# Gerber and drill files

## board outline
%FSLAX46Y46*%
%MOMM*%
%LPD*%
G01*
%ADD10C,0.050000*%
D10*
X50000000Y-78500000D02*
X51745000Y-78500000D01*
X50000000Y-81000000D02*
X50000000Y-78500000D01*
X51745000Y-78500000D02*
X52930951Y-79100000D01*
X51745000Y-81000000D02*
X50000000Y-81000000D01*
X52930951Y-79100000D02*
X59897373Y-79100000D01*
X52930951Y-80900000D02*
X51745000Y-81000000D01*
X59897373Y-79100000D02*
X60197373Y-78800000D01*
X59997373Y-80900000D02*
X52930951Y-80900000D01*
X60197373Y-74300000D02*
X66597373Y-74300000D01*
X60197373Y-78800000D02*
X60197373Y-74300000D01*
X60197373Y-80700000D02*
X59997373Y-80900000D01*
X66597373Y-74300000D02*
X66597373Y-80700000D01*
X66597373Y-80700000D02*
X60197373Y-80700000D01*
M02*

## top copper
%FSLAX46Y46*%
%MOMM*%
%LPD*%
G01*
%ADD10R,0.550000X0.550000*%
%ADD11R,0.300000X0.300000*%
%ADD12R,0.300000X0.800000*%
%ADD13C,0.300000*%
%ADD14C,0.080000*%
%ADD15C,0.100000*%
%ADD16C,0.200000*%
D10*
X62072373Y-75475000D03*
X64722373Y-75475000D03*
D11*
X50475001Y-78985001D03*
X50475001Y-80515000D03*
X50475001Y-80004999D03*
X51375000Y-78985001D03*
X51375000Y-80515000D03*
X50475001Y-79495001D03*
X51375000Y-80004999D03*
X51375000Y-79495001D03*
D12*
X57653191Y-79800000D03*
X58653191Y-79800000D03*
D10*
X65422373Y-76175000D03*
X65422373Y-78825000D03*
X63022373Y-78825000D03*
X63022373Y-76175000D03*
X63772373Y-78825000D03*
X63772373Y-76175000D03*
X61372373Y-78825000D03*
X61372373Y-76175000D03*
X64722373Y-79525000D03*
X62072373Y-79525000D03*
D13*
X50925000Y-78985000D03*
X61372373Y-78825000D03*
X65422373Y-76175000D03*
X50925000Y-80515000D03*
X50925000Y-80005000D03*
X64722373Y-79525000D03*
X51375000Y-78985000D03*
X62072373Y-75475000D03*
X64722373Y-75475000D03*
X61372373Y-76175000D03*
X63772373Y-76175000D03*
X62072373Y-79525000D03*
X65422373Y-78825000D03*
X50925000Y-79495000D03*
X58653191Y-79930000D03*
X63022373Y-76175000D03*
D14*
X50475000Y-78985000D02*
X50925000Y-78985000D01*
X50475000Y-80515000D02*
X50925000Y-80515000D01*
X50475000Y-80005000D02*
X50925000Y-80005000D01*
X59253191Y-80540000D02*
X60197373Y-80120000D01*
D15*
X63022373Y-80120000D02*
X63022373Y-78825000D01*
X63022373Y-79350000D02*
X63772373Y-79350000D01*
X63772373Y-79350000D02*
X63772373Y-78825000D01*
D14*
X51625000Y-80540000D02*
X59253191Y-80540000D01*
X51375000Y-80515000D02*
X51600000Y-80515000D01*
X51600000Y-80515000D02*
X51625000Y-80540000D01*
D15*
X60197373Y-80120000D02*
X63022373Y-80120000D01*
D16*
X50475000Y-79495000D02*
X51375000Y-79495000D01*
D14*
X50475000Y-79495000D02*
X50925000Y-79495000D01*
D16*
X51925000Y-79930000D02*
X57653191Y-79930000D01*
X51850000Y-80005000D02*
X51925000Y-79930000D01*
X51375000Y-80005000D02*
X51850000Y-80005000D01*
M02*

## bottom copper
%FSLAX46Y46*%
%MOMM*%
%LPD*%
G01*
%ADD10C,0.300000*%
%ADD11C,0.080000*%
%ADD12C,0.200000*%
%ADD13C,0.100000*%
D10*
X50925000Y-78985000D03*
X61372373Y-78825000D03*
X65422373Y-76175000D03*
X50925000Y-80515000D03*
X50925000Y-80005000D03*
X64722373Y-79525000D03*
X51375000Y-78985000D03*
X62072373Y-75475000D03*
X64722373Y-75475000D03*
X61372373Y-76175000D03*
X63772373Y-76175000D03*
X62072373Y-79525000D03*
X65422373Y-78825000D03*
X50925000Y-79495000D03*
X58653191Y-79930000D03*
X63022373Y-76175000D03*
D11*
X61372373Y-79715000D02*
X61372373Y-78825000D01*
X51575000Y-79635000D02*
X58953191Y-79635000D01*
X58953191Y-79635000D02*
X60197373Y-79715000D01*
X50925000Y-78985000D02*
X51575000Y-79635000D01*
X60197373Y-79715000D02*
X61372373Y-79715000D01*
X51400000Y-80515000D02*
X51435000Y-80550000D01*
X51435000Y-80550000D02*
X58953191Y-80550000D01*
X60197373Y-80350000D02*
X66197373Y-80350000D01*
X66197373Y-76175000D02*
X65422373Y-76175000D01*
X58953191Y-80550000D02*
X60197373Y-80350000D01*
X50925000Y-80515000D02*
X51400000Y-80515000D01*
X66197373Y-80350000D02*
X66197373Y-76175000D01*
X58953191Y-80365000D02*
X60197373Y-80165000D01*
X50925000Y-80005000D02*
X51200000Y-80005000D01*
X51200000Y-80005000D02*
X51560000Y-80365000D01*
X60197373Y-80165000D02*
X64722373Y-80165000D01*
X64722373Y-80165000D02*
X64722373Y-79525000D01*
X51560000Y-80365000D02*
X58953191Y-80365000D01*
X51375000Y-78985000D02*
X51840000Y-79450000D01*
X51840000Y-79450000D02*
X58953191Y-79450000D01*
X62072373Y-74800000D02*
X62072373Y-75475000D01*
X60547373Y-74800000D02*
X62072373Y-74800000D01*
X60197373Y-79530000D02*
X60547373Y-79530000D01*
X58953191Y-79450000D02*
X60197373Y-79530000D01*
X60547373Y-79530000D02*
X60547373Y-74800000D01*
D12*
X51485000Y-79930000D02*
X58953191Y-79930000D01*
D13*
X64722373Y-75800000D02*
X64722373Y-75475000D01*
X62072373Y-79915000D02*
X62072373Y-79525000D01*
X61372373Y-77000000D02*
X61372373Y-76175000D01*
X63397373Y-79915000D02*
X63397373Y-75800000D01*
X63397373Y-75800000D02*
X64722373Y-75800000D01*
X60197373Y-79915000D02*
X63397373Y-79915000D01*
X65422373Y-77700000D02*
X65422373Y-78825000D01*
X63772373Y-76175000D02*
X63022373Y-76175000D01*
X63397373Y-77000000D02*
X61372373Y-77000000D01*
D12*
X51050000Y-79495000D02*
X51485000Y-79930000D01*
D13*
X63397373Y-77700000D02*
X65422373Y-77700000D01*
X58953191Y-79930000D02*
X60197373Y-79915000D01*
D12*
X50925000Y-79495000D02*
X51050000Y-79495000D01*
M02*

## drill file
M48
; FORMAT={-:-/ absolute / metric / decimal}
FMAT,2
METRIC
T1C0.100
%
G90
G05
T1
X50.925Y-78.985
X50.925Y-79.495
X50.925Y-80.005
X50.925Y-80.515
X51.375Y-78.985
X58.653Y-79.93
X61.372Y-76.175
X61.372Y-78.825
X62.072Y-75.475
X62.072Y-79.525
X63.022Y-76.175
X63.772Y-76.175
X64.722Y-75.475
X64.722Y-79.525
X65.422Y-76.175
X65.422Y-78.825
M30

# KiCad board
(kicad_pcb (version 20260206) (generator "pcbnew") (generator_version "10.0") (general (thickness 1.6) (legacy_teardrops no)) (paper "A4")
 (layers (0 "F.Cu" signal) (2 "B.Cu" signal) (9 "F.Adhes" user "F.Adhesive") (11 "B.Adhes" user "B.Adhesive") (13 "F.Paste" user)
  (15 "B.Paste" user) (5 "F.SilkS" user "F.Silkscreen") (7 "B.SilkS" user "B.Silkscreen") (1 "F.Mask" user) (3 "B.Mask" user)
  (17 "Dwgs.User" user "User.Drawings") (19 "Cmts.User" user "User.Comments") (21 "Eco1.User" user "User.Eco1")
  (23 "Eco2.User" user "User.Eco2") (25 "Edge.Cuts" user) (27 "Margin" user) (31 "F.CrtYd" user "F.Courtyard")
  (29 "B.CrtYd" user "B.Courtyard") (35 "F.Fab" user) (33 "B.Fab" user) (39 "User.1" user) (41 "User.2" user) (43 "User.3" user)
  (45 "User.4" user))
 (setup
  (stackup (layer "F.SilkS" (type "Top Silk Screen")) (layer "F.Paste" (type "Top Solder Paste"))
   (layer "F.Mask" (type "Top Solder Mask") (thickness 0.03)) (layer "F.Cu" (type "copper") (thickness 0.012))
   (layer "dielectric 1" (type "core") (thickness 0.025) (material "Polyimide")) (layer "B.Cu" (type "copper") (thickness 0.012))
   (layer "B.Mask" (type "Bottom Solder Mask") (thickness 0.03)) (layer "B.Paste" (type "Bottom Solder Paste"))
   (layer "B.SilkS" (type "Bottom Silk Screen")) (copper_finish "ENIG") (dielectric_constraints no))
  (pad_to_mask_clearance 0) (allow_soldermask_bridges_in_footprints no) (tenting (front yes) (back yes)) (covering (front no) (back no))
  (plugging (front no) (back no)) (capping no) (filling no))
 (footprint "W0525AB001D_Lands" (layer "F.Cu") (at 58.153191 79.93)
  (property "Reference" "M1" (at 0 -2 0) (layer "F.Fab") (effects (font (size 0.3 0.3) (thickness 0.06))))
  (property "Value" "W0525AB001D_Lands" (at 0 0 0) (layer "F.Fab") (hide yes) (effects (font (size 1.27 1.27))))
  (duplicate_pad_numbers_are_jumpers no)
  (pad "1" smd rect (at -0.5 -0.13) (size 0.3 0.8) (layers "F.Cu" "F.Mask") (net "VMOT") (solder_mask_margin 0.05) (thermal_bridge_angle 45))
  (pad "2" smd rect (at 0.5 -0.13) (size 0.3 0.8) (layers "F.Cu" "F.Mask") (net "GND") (solder_mask_margin 0.05) (thermal_bridge_angle 45)))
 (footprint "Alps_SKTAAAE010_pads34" (layer "F.Cu") (at 63.397373 79.9 180)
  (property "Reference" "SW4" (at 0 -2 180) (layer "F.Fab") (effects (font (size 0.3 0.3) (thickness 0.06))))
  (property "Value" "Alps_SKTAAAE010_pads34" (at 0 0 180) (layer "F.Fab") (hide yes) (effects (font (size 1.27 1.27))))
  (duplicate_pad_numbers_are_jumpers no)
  (pad "3" smd rect (at -1.325 0.375 180) (size 0.55 0.55) (layers "F.Cu" "F.Mask" "F.Paste") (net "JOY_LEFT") (solder_mask_margin 0.05)
   (thermal_bridge_angle 45))
  (pad "4" smd rect (at 1.325 0.375 180) (size 0.55 0.55) (layers "F.Cu" "F.Mask" "F.Paste") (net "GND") (solder_mask_margin 0.05)
   (thermal_bridge_angle 45)))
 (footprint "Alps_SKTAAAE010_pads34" (layer "F.Cu") (at 60.997373 77.5 90)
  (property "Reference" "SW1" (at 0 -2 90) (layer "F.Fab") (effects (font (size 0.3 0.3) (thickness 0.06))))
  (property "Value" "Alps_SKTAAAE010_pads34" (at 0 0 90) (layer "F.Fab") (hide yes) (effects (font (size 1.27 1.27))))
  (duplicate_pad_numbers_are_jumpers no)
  (pad "3" smd rect (at -1.325 0.375 90) (size 0.55 0.55) (layers "F.Cu" "F.Mask" "F.Paste") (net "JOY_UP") (solder_mask_margin 0.05)
   (thermal_bridge_angle 45))
  (pad "4" smd rect (at 1.325 0.375 90) (size 0.55 0.55) (layers "F.Cu" "F.Mask" "F.Paste") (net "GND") (solder_mask_margin 0.05)
   (thermal_bridge_angle 45)))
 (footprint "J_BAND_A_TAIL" (layer "F.Cu") (at 50.9 79.75)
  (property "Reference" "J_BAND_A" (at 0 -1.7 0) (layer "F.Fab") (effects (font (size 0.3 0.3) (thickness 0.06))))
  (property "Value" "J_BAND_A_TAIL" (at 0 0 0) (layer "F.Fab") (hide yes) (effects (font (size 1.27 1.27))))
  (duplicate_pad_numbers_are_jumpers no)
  (pad "1" smd rect (at -0.424999 -0.764999) (size 0.3 0.3) (layers "F.Cu" "F.Mask") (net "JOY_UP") (solder_mask_margin 0.05)
   (thermal_bridge_angle 45))
  (pad "2" smd rect (at -0.424999 0.765) (size 0.3 0.3) (layers "F.Cu" "F.Mask") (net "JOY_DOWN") (solder_mask_margin 0.05)
   (thermal_bridge_angle 45))
  (pad "3" smd rect (at -0.424999 0.254999) (size 0.3 0.3) (layers "F.Cu" "F.Mask") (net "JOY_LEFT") (solder_mask_margin 0.05)
   (thermal_bridge_angle 45))
  (pad "4" smd rect (at 0.475 -0.764999) (size 0.3 0.3) (layers "F.Cu" "F.Mask") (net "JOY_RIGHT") (solder_mask_margin 0.05)
   (thermal_bridge_angle 45))
  (pad "5" smd rect (at 0.475 0.765) (size 0.3 0.3) (layers "F.Cu" "F.Mask") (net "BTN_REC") (solder_mask_margin 0.05)
   (thermal_bridge_angle 45))
  (pad "6" smd rect (at -0.424999 -0.254999) (size 0.3 0.3) (layers "F.Cu" "F.Mask") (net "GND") (solder_mask_margin 0.05)
   (thermal_bridge_angle 45))
  (pad "7" smd rect (at 0.475 0.254999) (size 0.3 0.3) (layers "F.Cu" "F.Mask") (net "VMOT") (solder_mask_margin 0.05)
   (thermal_bridge_angle 45))
  (pad "8" smd rect (at 0.475 -0.254999) (size 0.3 0.3) (layers "F.Cu" "F.Mask") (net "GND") (solder_mask_margin 0.05)
   (thermal_bridge_angle 45)))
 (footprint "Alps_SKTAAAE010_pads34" (layer "F.Cu") (at 65.797373 77.5 -90)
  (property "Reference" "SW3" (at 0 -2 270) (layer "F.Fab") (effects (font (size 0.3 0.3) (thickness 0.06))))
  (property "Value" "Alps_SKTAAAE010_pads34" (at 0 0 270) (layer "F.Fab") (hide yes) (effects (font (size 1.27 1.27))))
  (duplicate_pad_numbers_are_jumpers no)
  (pad "3" smd rect (at -1.325 0.375 270) (size 0.55 0.55) (layers "F.Cu" "F.Mask" "F.Paste") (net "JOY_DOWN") (solder_mask_margin 0.05)
   (thermal_bridge_angle 45))
  (pad "4" smd rect (at 1.325 0.375 270) (size 0.55 0.55) (layers "F.Cu" "F.Mask" "F.Paste") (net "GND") (solder_mask_margin 0.05)
   (thermal_bridge_angle 45)))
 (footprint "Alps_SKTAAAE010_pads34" (layer "F.Cu") (at 63.397373 75.1)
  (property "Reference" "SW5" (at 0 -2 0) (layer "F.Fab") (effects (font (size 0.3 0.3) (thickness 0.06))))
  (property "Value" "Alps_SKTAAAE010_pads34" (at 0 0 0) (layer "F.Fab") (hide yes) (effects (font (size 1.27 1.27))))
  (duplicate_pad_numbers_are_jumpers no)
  (pad "3" smd rect (at -1.325 0.375) (size 0.55 0.55) (layers "F.Cu" "F.Mask" "F.Paste") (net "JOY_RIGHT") (solder_mask_margin 0.05)
   (thermal_bridge_angle 45))
  (pad "4" smd rect (at 1.325 0.375) (size 0.55 0.55) (layers "F.Cu" "F.Mask" "F.Paste") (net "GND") (solder_mask_margin 0.05)
   (thermal_bridge_angle 45)))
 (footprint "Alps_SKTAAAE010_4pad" (layer "F.Cu") (at 63.397373 77.5 90)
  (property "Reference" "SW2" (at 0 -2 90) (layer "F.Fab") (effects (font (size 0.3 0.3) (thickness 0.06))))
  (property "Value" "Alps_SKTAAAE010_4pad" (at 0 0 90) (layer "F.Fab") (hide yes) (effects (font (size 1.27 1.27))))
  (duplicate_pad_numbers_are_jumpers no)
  (pad "1" smd rect (at -1.325 -0.375 90) (size 0.55 0.55) (layers "F.Cu" "F.Mask" "F.Paste") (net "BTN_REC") (solder_mask_margin 0.05)
   (thermal_bridge_angle 45))
  (pad "2" smd rect (at 1.325 -0.375 90) (size 0.55 0.55) (layers "F.Cu" "F.Mask" "F.Paste") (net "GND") (solder_mask_margin 0.05)
   (thermal_bridge_angle 45))
  (pad "3" smd rect (at -1.325 0.375 90) (size 0.55 0.55) (layers "F.Cu" "F.Mask" "F.Paste") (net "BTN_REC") (solder_mask_margin 0.05)
   (thermal_bridge_angle 45))
  (pad "4" smd rect (at 1.325 0.375 90) (size 0.55 0.55) (layers "F.Cu" "F.Mask" "F.Paste") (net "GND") (solder_mask_margin 0.05)
   (thermal_bridge_angle 45)))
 (gr_line (start 50 78.5) (end 51.745 78.5) (stroke (width 0.05) (type default)) (layer "Edge.Cuts"))
 (gr_line (start 50 81) (end 50 78.5) (stroke (width 0.05) (type default)) (layer "Edge.Cuts"))
 (gr_line (start 51.745 78.5) (end 52.930951 79.1) (stroke (width 0.05) (type default)) (layer "Edge.Cuts"))
 (gr_line (start 51.745 81) (end 50 81) (stroke (width 0.05) (type default)) (layer "Edge.Cuts"))
 (gr_line (start 52.930951 79.1) (end 59.897373 79.1) (stroke (width 0.05) (type default)) (layer "Edge.Cuts"))
 (gr_line (start 52.930951 80.9) (end 51.745 81) (stroke (width 0.05) (type default)) (layer "Edge.Cuts"))
 (gr_line (start 59.897373 79.1) (end 60.197373 78.8) (stroke (width 0.05) (type default)) (layer "Edge.Cuts"))
 (gr_line (start 59.997373 80.9) (end 52.930951 80.9) (stroke (width 0.05) (type default)) (layer "Edge.Cuts"))
 (gr_line (start 60.197373 74.3) (end 66.597373 74.3) (stroke (width 0.05) (type default)) (layer "Edge.Cuts"))
 (gr_line (start 60.197373 78.8) (end 60.197373 74.3) (stroke (width 0.05) (type default)) (layer "Edge.Cuts"))
 (gr_line (start 60.197373 80.7) (end 59.997373 80.9) (stroke (width 0.05) (type default)) (layer "Edge.Cuts"))
 (gr_line (start 66.597373 74.3) (end 66.597373 80.7) (stroke (width 0.05) (type default)) (layer "Edge.Cuts"))
 (gr_line (start 66.597373 80.7) (end 60.197373 80.7) (stroke (width 0.05) (type default)) (layer "Edge.Cuts"))
 (segment (start 50.475 78.985) (end 50.925 78.985) (width 0.08) (layer "F.Cu") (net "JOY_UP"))
 (via (at 61.372373 78.825) (size 0.3) (drill 0.1) (layers "F.Cu" "B.Cu") (tenting (front yes) (back yes)) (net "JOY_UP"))
 (via (at 50.925 78.985) (size 0.3) (drill 0.1) (layers "F.Cu" "B.Cu") (tenting (front yes) (back yes)) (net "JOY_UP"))
 (segment (start 58.953191 79.635) (end 60.197373 79.715) (width 0.08) (layer "B.Cu") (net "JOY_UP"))
 (segment (start 60.197373 79.715) (end 61.372373 79.715) (width 0.08) (layer "B.Cu") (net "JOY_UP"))
 (segment (start 50.925 78.985) (end 51.575 79.635) (width 0.08) (layer "B.Cu") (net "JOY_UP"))
 (segment (start 61.372373 79.715) (end 61.372373 78.825) (width 0.08) (layer "B.Cu") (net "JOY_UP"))
 (segment (start 51.575 79.635) (end 58.953191 79.635) (width 0.08) (layer "B.Cu") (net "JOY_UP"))
 (segment (start 50.475 80.515) (end 50.925 80.515) (width 0.08) (layer "F.Cu") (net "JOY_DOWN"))
 (via (at 65.422373 76.175) (size 0.3) (drill 0.1) (layers "F.Cu" "B.Cu") (tenting (front yes) (back yes)) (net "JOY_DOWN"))
 (via (at 50.925 80.515) (size 0.3) (drill 0.1) (layers "F.Cu" "B.Cu") (tenting (front yes) (back yes)) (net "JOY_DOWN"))
 (segment (start 58.953191 80.55) (end 60.197373 80.35) (width 0.08) (layer "B.Cu") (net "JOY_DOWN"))
 (segment (start 51.435 80.55) (end 58.953191 80.55) (width 0.08) (layer "B.Cu") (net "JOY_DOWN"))
 (segment (start 66.197373 80.35) (end 66.197373 76.175) (width 0.08) (layer "B.Cu") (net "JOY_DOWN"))
 (segment (start 50.925 80.515) (end 51.4 80.515) (width 0.08) (layer "B.Cu") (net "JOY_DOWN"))
 (segment (start 51.4 80.515) (end 51.435 80.55) (width 0.08) (layer "B.Cu") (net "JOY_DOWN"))
 (segment (start 60.197373 80.35) (end 66.197373 80.35) (width 0.08) (layer "B.Cu") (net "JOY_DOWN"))
 (segment (start 66.197373 76.175) (end 65.422373 76.175) (width 0.08) (layer "B.Cu") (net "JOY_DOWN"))
 (segment (start 50.475 80.005) (end 50.925 80.005) (width 0.08) (layer "F.Cu") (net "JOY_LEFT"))
 (via (at 64.722373 79.525) (size 0.3) (drill 0.1) (layers "F.Cu" "B.Cu") (tenting (front yes) (back yes)) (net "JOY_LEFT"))
 (via (at 50.925 80.005) (size 0.3) (drill 0.1) (layers "F.Cu" "B.Cu") (tenting (front yes) (back yes)) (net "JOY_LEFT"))
 (segment (start 51.56 80.365) (end 58.953191 80.365) (width 0.08) (layer "B.Cu") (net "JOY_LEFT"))
 (segment (start 64.722373 80.165) (end 64.722373 79.525) (width 0.08) (layer "B.Cu") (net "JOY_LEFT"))
 (segment (start 60.197373 80.165) (end 64.722373 80.165) (width 0.08) (layer "B.Cu") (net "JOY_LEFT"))
 (segment (start 58.953191 80.365) (end 60.197373 80.165) (width 0.08) (layer "B.Cu") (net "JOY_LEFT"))
 (segment (start 50.925 80.005) (end 51.2 80.005) (width 0.08) (layer "B.Cu") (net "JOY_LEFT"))
 (segment (start 51.2 80.005) (end 51.56 80.365) (width 0.08) (layer "B.Cu") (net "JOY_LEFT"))
 (via (at 62.072373 75.475) (size 0.3) (drill 0.1) (layers "F.Cu" "B.Cu") (tenting (front yes) (back yes)) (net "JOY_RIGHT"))
 (via (at 51.375 78.985) (size 0.3) (drill 0.1) (layers "F.Cu" "B.Cu") (tenting (front yes) (back yes)) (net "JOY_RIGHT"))
 (segment (start 60.547373 74.8) (end 62.072373 74.8) (width 0.08) (layer "B.Cu") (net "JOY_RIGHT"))
 (segment (start 60.547373 79.53) (end 60.547373 74.8) (width 0.08) (layer "B.Cu") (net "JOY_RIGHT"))
 (segment (start 51.375 78.985) (end 51.84 79.45) (width 0.08) (layer "B.Cu") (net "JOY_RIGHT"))
 (segment (start 62.072373 74.8) (end 62.072373 75.475) (width 0.08) (layer "B.Cu") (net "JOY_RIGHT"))
 (segment (start 51.84 79.45) (end 58.953191 79.45) (width 0.08) (layer "B.Cu") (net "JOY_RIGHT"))
 (segment (start 58.953191 79.45) (end 60.197373 79.53) (width 0.08) (layer "B.Cu") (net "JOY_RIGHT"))
 (segment (start 60.197373 79.53) (end 60.547373 79.53) (width 0.08) (layer "B.Cu") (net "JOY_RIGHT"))
 (segment (start 51.375 80.515) (end 51.6 80.515) (width 0.08) (layer "F.Cu") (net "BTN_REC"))
 (segment (start 63.022373 80.12) (end 63.022373 78.825) (width 0.1) (layer "F.Cu") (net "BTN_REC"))
 (segment (start 63.772373 79.35) (end 63.772373 78.825) (width 0.1) (layer "F.Cu") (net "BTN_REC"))
 (segment (start 63.022373 79.35) (end 63.772373 79.35) (width 0.1) (layer "F.Cu") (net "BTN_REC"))
 (segment (start 60.197373 80.12) (end 63.022373 80.12) (width 0.1) (layer "F.Cu") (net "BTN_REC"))
 (segment (start 59.253191 80.54) (end 60.197373 80.12) (width 0.08) (layer "F.Cu") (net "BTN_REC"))
 (segment (start 51.6 80.515) (end 51.625 80.54) (width 0.08) (layer "F.Cu") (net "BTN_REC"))
 (segment (start 51.625 80.54) (end 59.253191 80.54) (width 0.08) (layer "F.Cu") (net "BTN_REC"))
 (segment (start 50.475 79.495) (end 51.375 79.495) (width 0.2) (layer "F.Cu") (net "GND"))
 (segment (start 50.475 79.495) (end 50.925 79.495) (width 0.08) (layer "F.Cu") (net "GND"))
 (via (at 63.772373 76.175) (size 0.3) (drill 0.1) (layers "F.Cu" "B.Cu") (tenting (front yes) (back yes)) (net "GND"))
 (via (at 63.022373 76.175) (size 0.3) (drill 0.1) (layers "F.Cu" "B.Cu") (tenting (front yes) (back yes)) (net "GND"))
 (via (at 58.653191 79.93) (size 0.3) (drill 0.1) (layers "F.Cu" "B.Cu") (tenting (front yes) (back yes)) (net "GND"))
 (via (at 65.422373 78.825) (size 0.3) (drill 0.1) (layers "F.Cu" "B.Cu") (tenting (front yes) (back yes)) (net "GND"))
 (via (at 61.372373 76.175) (size 0.3) (drill 0.1) (layers "F.Cu" "B.Cu") (tenting (front yes) (back yes)) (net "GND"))
 (via (at 50.925 79.495) (size 0.3) (drill 0.1) (layers "F.Cu" "B.Cu") (tenting (front yes) (back yes)) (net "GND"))
 (via (at 62.072373 79.525) (size 0.3) (drill 0.1) (layers "F.Cu" "B.Cu") (tenting (front yes) (back yes)) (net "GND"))
 (via (at 64.722373 75.475) (size 0.3) (drill 0.1) (layers "F.Cu" "B.Cu") (tenting (front yes) (back yes)) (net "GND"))
 (segment (start 51.485 79.93) (end 58.953191 79.93) (width 0.2) (layer "B.Cu") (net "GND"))
 (segment (start 64.722373 75.8) (end 64.722373 75.475) (width 0.1) (layer "B.Cu") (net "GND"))
 (segment (start 63.397373 77.7) (end 65.422373 77.7) (width 0.1) (layer "B.Cu") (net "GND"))
 (segment (start 62.072373 79.915) (end 62.072373 79.525) (width 0.1) (layer "B.Cu") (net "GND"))
 (segment (start 63.397373 79.915) (end 63.397373 75.8) (width 0.1) (layer "B.Cu") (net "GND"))
 (segment (start 58.953191 79.93) (end 60.197373 79.915) (width 0.1) (layer "B.Cu") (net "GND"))
 (segment (start 65.422373 77.7) (end 65.422373 78.825) (width 0.1) (layer "B.Cu") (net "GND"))
 (segment (start 63.772373 76.175) (end 63.022373 76.175) (width 0.1) (layer "B.Cu") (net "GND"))
 (segment (start 63.397373 75.8) (end 64.722373 75.8) (width 0.1) (layer "B.Cu") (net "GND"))
 (segment (start 63.397373 77) (end 61.372373 77) (width 0.1) (layer "B.Cu") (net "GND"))
 (segment (start 61.372373 77) (end 61.372373 76.175) (width 0.1) (layer "B.Cu") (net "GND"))
 (segment (start 50.925 79.495) (end 51.05 79.495) (width 0.2) (layer "B.Cu") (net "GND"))
 (segment (start 60.197373 79.915) (end 63.397373 79.915) (width 0.1) (layer "B.Cu") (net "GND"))
 (segment (start 51.05 79.495) (end 51.485 79.93) (width 0.2) (layer "B.Cu") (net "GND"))
 (segment (start 51.925 79.93) (end 57.653191 79.93) (width 0.2) (layer "F.Cu") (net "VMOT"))
 (segment (start 51.375 80.005) (end 51.85 80.005) (width 0.2) (layer "F.Cu") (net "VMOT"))
 (segment (start 51.85 80.005) (end 51.925 79.93) (width 0.2) (layer "F.Cu") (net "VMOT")))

